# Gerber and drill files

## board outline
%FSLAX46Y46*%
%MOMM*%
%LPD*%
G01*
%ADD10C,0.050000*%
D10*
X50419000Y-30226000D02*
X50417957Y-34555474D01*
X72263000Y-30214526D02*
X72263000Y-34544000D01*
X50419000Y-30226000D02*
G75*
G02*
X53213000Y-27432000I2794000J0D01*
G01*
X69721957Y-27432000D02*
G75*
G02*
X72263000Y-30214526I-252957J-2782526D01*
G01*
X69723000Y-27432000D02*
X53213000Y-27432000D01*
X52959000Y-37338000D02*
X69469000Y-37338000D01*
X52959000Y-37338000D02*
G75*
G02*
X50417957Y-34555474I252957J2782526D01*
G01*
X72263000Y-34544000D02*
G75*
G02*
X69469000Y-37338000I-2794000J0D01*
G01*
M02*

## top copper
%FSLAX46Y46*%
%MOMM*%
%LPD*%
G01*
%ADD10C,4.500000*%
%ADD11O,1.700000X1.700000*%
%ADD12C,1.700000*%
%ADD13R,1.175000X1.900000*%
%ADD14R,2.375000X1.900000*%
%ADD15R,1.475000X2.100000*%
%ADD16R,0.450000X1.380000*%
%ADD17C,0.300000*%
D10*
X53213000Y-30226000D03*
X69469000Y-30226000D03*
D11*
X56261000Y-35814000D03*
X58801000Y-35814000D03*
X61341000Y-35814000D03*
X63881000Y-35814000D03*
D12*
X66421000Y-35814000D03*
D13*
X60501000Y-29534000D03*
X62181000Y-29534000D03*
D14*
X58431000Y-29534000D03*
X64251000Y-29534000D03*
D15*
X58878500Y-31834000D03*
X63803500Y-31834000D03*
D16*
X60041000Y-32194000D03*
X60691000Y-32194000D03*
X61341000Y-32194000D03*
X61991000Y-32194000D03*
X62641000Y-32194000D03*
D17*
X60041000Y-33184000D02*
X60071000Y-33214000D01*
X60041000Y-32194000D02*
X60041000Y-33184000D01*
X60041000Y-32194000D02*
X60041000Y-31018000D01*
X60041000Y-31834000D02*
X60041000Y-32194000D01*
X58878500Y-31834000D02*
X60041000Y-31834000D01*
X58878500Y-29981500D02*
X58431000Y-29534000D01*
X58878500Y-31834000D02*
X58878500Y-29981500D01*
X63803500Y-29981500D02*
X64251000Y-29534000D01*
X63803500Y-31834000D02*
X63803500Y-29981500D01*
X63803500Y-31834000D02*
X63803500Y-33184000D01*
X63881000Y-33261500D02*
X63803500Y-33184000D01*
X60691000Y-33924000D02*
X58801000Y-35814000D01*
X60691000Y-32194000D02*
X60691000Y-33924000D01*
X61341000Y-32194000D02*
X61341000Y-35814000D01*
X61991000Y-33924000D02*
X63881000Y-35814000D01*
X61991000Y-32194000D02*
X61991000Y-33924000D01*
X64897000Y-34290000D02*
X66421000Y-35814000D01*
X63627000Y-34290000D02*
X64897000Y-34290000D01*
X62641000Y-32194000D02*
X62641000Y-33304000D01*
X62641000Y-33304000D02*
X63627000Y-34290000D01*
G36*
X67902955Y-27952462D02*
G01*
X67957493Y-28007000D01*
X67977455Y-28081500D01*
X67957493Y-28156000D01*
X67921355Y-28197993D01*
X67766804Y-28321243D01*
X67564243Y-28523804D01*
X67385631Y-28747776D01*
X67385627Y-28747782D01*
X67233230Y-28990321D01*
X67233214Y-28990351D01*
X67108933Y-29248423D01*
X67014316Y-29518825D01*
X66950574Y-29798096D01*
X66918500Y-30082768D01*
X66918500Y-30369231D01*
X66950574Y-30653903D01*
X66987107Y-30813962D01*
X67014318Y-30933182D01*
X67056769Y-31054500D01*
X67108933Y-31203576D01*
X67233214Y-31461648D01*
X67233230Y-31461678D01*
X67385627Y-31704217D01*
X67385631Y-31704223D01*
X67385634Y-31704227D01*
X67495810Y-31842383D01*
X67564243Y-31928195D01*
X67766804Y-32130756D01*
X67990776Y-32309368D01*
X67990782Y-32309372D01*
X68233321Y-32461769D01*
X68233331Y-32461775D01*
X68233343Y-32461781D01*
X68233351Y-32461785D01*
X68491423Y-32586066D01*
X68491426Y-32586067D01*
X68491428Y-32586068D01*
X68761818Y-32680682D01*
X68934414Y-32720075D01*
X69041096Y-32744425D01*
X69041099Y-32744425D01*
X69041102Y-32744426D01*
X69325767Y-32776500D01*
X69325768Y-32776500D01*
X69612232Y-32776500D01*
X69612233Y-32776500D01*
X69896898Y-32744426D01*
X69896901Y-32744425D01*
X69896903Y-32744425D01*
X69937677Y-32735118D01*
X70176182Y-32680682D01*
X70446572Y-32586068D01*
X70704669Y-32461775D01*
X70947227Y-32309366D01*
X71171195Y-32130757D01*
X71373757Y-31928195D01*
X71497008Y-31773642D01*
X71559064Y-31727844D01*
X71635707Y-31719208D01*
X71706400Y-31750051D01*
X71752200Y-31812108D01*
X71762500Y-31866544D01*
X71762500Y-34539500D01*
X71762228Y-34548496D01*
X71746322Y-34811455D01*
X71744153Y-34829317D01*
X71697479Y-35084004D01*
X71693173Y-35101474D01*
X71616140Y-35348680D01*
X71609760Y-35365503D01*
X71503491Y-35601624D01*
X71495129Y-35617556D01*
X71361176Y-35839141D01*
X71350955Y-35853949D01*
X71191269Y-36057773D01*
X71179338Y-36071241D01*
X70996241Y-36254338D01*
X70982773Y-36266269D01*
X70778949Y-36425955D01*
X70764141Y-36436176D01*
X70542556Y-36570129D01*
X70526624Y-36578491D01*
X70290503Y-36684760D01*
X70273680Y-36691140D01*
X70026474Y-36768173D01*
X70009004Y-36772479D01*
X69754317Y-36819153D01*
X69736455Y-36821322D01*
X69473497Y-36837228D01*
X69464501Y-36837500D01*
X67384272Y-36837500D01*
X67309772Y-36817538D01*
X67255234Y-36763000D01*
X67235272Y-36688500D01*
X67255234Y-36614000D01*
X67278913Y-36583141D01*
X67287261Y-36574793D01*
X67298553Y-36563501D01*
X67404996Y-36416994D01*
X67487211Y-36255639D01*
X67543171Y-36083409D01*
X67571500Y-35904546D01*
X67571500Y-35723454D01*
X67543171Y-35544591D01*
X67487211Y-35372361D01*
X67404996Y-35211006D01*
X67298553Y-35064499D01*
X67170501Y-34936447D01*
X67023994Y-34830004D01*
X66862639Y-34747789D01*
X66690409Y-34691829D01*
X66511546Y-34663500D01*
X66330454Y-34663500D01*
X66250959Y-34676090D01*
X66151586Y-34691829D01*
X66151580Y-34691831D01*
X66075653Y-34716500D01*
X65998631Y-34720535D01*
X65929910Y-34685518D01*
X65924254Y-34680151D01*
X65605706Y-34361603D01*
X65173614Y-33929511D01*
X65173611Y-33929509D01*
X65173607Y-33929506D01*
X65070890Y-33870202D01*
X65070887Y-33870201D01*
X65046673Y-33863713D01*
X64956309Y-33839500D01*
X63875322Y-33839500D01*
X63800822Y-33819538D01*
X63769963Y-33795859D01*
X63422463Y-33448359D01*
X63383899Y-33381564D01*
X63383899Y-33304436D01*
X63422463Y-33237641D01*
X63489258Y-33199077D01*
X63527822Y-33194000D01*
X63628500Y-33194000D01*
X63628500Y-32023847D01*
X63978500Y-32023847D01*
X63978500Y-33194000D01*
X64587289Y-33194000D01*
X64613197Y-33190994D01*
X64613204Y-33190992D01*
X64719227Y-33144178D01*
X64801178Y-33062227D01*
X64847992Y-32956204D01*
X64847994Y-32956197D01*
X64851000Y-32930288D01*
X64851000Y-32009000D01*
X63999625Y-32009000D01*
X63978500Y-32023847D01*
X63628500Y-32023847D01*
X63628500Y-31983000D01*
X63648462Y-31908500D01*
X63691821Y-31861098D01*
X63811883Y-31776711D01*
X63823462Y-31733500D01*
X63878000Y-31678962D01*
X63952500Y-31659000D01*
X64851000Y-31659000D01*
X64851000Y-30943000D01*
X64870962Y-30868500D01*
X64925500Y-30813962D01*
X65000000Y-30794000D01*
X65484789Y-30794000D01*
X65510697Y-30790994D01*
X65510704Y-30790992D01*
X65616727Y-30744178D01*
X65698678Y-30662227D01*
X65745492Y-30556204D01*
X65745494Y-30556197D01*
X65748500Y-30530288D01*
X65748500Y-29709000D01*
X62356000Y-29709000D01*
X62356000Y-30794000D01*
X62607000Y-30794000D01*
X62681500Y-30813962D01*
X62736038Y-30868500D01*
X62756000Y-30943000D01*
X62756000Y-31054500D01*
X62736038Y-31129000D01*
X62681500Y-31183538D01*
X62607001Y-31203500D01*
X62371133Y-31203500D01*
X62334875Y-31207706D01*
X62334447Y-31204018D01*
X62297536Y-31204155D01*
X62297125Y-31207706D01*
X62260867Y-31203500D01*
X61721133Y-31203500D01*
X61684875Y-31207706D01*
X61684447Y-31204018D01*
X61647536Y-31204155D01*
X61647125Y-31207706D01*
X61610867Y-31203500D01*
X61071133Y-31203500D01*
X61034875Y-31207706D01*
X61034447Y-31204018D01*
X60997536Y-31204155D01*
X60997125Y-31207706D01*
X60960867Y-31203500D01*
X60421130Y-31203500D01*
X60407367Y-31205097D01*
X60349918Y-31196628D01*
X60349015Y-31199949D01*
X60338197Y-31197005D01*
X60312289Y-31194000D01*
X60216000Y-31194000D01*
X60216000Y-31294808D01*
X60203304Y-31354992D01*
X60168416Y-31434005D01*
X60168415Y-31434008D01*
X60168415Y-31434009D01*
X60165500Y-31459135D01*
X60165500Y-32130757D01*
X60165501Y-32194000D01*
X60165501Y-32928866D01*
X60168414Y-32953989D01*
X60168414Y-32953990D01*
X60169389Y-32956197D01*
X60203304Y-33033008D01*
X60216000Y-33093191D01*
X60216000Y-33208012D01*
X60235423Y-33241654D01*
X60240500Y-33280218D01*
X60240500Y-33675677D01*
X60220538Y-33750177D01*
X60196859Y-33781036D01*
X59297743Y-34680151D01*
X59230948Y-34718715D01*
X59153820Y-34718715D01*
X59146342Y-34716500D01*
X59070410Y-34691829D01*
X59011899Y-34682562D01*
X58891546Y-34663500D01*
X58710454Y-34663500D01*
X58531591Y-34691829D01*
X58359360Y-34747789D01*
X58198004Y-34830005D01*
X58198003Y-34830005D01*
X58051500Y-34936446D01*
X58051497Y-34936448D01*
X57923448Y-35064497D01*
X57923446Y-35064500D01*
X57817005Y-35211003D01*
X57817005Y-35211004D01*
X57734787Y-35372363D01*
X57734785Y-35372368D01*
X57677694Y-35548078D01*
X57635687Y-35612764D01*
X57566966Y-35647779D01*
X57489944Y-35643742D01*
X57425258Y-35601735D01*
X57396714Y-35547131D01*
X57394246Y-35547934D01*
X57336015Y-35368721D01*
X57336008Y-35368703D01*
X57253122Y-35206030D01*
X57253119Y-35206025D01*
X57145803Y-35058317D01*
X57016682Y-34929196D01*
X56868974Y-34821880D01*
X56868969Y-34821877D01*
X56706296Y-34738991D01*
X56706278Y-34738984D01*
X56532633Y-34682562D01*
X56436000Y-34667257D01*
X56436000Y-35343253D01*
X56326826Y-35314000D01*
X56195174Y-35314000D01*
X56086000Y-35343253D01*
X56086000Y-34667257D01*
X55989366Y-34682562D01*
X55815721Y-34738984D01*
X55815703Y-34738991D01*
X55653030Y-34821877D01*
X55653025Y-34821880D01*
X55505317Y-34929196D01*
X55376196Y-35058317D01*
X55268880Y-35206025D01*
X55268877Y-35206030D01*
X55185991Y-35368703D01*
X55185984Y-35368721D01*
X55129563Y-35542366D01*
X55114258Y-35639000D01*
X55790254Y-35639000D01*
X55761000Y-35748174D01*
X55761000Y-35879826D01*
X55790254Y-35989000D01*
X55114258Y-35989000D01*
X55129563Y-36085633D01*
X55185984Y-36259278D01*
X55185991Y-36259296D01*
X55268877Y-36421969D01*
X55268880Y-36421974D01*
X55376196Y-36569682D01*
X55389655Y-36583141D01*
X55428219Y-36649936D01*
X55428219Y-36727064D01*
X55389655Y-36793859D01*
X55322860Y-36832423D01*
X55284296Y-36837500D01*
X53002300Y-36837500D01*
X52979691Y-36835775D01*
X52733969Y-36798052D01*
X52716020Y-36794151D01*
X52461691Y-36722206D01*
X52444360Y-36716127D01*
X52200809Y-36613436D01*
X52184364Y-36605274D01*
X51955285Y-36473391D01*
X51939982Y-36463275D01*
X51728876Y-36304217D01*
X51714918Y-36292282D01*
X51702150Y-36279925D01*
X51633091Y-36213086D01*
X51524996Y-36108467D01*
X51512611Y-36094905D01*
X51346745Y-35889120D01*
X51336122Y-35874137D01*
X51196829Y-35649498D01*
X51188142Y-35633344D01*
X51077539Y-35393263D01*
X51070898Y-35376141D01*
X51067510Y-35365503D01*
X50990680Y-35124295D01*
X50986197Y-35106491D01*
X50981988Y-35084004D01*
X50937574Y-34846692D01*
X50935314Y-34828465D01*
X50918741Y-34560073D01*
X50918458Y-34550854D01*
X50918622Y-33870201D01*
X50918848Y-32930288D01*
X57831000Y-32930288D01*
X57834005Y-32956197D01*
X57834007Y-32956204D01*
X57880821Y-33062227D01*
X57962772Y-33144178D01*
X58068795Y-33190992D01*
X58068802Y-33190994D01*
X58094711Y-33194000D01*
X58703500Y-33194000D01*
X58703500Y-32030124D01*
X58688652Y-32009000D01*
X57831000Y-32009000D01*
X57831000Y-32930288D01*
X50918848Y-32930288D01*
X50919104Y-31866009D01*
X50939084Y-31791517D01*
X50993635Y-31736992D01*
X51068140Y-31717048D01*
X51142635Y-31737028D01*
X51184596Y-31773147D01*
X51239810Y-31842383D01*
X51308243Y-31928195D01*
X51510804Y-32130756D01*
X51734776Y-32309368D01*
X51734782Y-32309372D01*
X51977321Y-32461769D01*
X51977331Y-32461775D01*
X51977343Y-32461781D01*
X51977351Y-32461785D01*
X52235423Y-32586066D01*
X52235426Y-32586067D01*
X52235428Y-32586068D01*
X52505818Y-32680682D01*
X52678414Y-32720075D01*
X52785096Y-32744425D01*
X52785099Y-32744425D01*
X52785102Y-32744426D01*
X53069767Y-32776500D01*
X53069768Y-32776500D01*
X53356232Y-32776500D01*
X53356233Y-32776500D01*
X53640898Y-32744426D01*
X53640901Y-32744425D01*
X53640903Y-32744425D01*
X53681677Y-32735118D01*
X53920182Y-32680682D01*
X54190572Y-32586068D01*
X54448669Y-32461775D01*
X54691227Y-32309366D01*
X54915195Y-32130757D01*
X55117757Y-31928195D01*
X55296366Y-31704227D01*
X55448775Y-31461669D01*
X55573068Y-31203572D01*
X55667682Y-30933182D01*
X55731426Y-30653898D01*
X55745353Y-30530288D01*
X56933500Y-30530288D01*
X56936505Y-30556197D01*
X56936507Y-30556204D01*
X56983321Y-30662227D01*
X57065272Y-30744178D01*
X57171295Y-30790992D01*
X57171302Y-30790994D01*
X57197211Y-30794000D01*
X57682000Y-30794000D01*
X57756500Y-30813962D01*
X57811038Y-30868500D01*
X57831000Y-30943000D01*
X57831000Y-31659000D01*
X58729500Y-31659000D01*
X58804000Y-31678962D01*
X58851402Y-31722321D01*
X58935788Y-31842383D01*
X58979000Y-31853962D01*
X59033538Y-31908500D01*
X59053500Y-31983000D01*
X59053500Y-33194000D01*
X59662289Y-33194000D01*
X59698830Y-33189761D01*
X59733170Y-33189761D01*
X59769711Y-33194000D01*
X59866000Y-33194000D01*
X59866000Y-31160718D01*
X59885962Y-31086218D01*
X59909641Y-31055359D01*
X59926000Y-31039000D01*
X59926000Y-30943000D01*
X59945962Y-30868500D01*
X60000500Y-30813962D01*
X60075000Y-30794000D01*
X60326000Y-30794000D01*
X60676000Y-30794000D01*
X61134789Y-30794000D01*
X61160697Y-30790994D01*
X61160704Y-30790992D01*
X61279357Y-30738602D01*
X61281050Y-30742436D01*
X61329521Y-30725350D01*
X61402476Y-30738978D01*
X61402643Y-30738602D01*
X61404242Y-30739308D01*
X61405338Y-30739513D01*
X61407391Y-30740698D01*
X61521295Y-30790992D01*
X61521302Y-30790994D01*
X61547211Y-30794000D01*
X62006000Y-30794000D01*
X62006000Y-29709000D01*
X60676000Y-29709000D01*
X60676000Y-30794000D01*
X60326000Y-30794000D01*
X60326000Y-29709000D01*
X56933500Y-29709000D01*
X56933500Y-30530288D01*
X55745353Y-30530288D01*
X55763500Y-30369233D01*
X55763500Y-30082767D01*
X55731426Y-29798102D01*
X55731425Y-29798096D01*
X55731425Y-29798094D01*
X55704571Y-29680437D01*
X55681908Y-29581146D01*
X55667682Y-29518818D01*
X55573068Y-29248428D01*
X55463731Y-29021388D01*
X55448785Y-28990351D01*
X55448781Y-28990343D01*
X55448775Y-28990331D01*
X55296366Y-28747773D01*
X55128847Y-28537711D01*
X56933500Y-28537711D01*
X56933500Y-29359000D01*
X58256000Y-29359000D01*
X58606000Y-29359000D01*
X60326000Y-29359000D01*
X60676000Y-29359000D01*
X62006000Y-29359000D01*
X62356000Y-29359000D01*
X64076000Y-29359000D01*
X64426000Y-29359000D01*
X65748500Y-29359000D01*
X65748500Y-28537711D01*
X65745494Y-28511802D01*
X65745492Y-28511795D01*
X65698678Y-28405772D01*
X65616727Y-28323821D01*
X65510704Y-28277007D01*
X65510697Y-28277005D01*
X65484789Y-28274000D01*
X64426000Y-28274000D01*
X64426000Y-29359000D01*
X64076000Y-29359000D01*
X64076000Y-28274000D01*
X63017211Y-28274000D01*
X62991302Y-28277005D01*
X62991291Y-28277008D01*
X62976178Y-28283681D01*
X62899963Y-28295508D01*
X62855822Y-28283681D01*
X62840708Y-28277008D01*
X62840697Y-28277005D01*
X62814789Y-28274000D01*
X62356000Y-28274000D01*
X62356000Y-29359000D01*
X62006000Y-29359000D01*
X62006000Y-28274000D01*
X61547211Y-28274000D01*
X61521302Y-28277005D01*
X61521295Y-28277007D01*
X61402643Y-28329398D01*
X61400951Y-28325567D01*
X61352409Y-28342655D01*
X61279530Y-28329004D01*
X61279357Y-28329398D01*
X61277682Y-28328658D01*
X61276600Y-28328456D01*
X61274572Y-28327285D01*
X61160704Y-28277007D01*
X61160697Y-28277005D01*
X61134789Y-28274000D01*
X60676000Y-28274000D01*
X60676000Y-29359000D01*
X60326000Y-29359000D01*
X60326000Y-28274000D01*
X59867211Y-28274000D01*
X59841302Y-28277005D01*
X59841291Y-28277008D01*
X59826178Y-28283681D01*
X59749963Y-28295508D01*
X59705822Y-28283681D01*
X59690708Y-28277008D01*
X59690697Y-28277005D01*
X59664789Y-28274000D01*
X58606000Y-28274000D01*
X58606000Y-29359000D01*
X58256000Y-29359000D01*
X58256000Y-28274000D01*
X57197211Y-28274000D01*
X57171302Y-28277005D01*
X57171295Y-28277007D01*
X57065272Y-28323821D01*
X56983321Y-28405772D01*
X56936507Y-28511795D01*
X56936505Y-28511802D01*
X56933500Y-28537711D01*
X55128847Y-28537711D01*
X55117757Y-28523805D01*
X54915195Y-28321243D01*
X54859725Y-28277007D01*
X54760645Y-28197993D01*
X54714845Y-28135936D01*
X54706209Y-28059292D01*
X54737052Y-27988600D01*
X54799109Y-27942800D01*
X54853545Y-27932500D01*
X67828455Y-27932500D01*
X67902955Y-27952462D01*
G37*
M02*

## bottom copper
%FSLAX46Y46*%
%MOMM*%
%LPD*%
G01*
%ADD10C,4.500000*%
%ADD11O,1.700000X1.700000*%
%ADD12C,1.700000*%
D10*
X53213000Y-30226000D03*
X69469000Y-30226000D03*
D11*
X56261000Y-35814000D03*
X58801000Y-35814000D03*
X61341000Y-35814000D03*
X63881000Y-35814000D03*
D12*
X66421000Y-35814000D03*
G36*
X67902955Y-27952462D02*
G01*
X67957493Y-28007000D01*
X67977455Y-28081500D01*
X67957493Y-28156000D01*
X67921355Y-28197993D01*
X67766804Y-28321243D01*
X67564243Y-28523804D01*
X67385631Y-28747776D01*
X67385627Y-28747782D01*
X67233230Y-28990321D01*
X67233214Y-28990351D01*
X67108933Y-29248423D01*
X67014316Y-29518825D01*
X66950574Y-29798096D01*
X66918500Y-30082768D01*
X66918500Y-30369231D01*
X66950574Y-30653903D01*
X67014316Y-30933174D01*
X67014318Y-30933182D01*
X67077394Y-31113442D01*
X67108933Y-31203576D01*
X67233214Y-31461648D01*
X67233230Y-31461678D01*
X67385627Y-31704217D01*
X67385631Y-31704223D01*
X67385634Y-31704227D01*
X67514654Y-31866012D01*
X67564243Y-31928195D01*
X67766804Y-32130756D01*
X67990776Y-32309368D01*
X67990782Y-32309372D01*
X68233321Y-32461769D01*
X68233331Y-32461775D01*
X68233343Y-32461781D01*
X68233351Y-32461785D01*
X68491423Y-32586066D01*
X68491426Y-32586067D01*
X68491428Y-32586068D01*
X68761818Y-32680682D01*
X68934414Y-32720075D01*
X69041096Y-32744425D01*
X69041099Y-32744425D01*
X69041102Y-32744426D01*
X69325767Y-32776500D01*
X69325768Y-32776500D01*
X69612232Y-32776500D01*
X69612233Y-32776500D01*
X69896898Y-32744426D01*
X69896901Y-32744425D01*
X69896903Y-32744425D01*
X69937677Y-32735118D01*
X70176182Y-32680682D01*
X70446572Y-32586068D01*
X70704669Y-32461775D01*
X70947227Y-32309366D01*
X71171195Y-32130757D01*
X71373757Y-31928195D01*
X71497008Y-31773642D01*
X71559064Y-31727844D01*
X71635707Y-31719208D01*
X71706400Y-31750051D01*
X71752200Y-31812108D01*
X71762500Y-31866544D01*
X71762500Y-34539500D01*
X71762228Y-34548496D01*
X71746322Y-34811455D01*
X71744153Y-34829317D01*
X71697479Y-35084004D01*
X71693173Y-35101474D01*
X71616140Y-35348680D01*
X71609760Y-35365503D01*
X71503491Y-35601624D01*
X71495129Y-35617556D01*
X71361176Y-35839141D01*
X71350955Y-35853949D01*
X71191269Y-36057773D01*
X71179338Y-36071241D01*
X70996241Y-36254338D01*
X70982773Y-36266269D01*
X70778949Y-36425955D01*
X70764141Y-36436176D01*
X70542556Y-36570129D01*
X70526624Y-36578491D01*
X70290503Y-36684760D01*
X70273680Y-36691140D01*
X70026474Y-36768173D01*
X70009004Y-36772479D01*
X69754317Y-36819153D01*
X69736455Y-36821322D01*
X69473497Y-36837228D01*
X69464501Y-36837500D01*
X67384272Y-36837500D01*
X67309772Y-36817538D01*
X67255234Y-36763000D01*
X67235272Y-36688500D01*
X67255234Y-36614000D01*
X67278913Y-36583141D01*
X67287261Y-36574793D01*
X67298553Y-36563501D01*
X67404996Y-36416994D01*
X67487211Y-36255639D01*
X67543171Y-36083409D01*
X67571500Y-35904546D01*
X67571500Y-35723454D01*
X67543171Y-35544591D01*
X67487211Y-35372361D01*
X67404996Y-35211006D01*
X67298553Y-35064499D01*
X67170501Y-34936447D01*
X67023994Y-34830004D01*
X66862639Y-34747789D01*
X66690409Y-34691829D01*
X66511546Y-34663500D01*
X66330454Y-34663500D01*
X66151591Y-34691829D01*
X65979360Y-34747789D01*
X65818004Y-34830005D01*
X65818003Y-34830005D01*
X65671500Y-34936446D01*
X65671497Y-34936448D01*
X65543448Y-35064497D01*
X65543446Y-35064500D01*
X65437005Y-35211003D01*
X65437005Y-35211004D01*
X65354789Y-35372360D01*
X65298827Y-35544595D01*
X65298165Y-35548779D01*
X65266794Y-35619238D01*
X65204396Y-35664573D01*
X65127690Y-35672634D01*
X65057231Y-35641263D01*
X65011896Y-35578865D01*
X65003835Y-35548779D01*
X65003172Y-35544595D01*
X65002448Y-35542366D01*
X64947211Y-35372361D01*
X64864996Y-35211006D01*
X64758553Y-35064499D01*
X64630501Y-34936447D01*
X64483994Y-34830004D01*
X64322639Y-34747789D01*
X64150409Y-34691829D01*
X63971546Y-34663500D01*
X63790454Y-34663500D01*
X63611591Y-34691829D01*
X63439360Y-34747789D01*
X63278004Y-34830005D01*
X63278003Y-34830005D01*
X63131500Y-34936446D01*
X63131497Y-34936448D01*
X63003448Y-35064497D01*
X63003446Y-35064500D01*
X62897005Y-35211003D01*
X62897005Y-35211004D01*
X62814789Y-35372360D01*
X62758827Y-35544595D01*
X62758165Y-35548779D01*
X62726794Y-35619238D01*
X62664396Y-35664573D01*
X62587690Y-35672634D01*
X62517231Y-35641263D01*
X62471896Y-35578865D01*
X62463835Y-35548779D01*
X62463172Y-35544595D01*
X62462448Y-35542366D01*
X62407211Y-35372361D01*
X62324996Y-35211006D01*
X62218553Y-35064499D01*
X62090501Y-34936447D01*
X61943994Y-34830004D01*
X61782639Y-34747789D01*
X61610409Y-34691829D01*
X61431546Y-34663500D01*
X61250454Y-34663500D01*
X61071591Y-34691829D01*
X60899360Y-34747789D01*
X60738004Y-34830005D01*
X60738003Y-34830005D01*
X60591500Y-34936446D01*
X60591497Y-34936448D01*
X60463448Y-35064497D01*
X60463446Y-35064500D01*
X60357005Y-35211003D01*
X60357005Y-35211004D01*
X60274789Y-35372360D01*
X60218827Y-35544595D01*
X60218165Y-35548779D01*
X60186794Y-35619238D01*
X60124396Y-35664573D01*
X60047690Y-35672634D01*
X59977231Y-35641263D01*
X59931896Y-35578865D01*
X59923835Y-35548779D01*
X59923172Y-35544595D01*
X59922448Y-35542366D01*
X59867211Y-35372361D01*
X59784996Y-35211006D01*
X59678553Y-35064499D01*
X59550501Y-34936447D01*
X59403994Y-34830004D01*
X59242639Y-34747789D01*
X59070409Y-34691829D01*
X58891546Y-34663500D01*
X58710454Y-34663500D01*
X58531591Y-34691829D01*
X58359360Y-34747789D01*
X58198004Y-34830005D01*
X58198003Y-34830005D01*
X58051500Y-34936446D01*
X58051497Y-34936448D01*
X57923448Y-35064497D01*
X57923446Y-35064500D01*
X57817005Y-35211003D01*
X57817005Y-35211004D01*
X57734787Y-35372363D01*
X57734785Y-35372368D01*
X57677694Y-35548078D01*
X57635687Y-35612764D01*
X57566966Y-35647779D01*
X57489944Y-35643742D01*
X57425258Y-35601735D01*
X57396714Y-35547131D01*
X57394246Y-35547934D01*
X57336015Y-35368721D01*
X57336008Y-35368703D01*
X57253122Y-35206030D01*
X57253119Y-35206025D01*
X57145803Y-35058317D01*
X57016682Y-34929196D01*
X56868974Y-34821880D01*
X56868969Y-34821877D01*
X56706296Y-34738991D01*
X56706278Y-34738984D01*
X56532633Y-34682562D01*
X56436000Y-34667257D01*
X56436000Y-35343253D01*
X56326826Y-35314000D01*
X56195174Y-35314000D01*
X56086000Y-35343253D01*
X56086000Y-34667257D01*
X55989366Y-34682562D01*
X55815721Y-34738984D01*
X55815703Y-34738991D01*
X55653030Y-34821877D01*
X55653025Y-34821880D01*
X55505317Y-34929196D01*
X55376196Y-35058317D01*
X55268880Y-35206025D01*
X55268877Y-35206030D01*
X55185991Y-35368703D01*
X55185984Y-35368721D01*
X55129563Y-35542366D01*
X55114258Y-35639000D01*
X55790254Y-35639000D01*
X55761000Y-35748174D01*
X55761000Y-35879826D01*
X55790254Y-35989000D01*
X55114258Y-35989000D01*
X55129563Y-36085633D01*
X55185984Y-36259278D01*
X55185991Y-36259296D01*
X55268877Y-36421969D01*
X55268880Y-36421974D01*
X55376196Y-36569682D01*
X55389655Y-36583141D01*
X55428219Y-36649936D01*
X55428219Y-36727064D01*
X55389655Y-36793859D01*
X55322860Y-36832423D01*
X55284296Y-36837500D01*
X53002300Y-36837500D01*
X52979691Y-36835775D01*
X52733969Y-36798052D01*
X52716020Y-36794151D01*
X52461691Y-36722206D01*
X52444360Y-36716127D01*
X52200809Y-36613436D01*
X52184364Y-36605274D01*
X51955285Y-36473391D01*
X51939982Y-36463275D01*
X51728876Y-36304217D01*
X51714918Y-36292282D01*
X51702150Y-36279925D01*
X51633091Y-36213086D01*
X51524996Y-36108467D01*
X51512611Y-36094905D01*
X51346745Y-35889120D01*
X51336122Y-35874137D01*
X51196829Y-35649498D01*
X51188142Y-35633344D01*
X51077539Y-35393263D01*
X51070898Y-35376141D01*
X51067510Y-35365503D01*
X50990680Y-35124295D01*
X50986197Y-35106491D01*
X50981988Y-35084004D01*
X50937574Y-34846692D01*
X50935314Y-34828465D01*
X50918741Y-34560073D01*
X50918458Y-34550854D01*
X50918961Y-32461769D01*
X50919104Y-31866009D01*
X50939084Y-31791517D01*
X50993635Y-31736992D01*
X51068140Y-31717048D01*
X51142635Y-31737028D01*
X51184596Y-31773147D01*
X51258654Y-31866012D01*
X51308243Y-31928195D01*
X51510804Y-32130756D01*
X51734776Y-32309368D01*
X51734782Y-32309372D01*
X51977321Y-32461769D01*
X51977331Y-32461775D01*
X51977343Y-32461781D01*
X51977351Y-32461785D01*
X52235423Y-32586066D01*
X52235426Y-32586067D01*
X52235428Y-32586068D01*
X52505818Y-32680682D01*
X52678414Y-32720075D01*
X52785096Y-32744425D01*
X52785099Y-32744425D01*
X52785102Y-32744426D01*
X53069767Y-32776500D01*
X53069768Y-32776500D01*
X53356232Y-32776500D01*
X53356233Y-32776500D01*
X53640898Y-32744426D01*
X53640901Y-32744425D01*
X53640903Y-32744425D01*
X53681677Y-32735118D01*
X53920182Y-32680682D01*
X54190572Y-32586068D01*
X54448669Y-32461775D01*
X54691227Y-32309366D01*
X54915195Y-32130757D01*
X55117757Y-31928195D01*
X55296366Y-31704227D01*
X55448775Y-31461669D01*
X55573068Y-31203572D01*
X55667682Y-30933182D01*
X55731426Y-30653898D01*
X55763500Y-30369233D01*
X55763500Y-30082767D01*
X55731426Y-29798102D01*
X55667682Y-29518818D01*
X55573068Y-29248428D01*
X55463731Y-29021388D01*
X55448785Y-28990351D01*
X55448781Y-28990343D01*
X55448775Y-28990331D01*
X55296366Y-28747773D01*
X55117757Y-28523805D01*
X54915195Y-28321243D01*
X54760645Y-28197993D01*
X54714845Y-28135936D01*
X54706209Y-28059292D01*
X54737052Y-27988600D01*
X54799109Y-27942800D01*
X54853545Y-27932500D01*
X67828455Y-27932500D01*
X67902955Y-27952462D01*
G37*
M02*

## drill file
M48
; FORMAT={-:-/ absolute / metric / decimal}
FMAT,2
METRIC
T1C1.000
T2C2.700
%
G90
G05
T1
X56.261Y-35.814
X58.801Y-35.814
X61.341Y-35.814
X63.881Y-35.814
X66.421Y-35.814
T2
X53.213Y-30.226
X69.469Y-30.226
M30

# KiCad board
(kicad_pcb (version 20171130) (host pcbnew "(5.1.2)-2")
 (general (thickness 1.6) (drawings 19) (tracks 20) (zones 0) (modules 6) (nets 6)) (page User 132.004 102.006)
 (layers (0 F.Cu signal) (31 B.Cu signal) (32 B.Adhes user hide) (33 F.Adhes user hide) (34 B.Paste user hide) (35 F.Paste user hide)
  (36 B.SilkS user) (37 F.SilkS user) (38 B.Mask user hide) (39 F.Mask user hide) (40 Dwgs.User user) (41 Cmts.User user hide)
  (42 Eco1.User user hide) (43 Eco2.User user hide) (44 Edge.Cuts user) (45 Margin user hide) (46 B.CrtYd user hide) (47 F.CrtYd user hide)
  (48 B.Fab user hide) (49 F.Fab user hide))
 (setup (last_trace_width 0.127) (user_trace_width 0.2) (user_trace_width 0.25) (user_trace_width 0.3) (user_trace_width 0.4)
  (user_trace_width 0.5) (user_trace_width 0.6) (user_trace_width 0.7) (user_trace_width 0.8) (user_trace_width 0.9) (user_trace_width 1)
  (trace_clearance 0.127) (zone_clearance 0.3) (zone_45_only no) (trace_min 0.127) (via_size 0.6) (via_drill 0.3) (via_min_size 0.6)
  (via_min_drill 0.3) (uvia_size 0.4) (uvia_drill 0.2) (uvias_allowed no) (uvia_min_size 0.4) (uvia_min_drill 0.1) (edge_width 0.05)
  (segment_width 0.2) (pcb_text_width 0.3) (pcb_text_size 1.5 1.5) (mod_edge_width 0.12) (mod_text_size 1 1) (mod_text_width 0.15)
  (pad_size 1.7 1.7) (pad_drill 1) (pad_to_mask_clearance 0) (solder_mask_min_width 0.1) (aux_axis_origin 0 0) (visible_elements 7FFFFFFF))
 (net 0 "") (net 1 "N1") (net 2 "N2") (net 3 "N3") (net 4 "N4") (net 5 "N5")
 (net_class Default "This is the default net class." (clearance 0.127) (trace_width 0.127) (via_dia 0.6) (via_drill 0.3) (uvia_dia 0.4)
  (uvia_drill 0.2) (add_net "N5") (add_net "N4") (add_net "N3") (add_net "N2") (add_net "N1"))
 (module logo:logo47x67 (layer B.Cu) (at 61.341 30.226 180)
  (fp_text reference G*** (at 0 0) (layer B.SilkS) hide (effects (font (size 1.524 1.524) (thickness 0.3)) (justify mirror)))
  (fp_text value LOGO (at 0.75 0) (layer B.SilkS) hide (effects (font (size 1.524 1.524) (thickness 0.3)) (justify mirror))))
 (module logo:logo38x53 (layer F.Cu) (at 53.213 34.798)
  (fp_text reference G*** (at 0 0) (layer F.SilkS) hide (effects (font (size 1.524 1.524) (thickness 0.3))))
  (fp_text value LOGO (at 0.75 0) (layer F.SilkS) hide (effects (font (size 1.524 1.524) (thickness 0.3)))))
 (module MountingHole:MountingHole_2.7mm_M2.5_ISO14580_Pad (layer F.Cu) (at 53.213 30.226 270)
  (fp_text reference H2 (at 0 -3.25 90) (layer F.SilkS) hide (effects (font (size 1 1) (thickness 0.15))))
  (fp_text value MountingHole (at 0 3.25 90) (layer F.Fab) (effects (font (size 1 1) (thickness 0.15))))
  (pad 1 thru_hole circle (at 0 0 270) (size 4.5 4.5) (drill 2.7) (layers *.Cu *.Mask)))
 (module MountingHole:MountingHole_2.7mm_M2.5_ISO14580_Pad (layer F.Cu) (at 69.469 30.226 270)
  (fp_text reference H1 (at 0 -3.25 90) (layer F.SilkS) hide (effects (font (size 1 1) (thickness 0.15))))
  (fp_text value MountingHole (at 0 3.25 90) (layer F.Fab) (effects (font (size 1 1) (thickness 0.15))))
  (pad 1 thru_hole circle (at 0 0 270) (size 4.5 4.5) (drill 2.7) (layers *.Cu *.Mask)))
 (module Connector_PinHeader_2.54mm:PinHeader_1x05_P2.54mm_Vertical (layer B.Cu) (at 66.421 35.814 90)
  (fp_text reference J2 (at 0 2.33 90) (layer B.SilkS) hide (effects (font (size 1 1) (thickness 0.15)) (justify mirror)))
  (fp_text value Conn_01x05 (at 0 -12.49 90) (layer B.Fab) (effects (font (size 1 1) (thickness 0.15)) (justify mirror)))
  (pad 5 thru_hole oval (at 0 -10.16 90) (size 1.7 1.7) (drill 1) (layers *.Cu *.Mask) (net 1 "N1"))
  (pad 4 thru_hole oval (at 0 -7.62 90) (size 1.7 1.7) (drill 1) (layers *.Cu *.Mask) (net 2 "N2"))
  (pad 3 thru_hole oval (at 0 -5.08 90) (size 1.7 1.7) (drill 1) (layers *.Cu *.Mask) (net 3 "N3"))
  (pad 2 thru_hole oval (at 0 -2.54 90) (size 1.7 1.7) (drill 1) (layers *.Cu *.Mask) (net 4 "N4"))
  (pad 1 thru_hole circle (at 0 0 90) (size 1.7 1.7) (drill 1) (layers *.Cu *.Mask) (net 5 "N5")))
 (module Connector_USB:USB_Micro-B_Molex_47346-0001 (layer F.Cu) (at 61.341 30.734 180)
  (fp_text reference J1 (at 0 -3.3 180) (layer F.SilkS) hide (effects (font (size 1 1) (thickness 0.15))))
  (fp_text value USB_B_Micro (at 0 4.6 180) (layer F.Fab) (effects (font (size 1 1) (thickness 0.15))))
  (pad 6 smd rect (at 0.84 1.2 180) (size 1.175 1.9) (layers F.Cu F.Paste F.Mask) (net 1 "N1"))
  (pad 6 smd rect (at -0.84 1.2 180) (size 1.175 1.9) (layers F.Cu F.Paste F.Mask) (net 1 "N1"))
  (pad 6 smd rect (at 2.91 1.2 180) (size 2.375 1.9) (layers F.Cu F.Paste F.Mask) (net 1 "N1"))
  (pad 6 smd rect (at -2.91 1.2 180) (size 2.375 1.9) (layers F.Cu F.Paste F.Mask) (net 1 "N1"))
  (pad 6 smd rect (at 2.4625 -1.1 180) (size 1.475 2.1) (layers F.Cu F.Paste F.Mask) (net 1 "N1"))
  (pad 6 smd rect (at -2.4625 -1.1 180) (size 1.475 2.1) (layers F.Cu F.Paste F.Mask) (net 1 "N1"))
  (pad 5 smd rect (at 1.3 -1.46 180) (size 0.45 1.38) (layers F.Cu F.Paste F.Mask) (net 1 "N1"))
  (pad 4 smd rect (at 0.65 -1.46 180) (size 0.45 1.38) (layers F.Cu F.Paste F.Mask) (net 2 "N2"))
  (pad 3 smd rect (at 0 -1.46 180) (size 0.45 1.38) (layers F.Cu F.Paste F.Mask) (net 3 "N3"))
  (pad 2 smd rect (at -0.65 -1.46 180) (size 0.45 1.38) (layers F.Cu F.Paste F.Mask) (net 4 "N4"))
  (pad 1 smd rect (at -1.3 -1.46 180) (size 0.45 1.38) (layers F.Cu F.Paste F.Mask) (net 5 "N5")))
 (gr_line (start 50.419 30.226) (end 50.417957 34.555474) (layer Edge.Cuts) (width 0.05))
 (gr_line (start 72.263 30.214526) (end 72.263 34.544) (layer Edge.Cuts) (width 0.05))
 (gr_arc (start 53.213 30.226) (end 53.213 27.432) (angle -90) (layer Edge.Cuts) (width 0.05))
 (gr_arc (start 69.469 30.214526) (end 72.263 30.214526) (angle -84.80557109) (layer Edge.Cuts) (width 0.05))
 (gr_line (start 69.723 27.432) (end 53.213 27.432) (layer Edge.Cuts) (width 0.05))
 (gr_line (start 52.959 37.338) (end 69.469 37.338) (layer Edge.Cuts) (width 0.05))
 (gr_arc (start 53.211957 34.555474) (end 50.417957 34.555474) (angle -84.80557109) (layer Edge.Cuts) (width 0.05))
 (gr_arc (start 69.469 34.544) (end 69.469 37.338) (angle -90) (layer Edge.Cuts) (width 0.05))
 (segment (start 60.041 33.184) (end 60.071 33.214) (width 0.3) (layer F.Cu) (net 1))
 (segment (start 60.041 32.194) (end 60.041 33.184) (width 0.3) (layer F.Cu) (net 1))
 (segment (start 60.041 32.194) (end 60.041 31.018) (width 0.3) (layer F.Cu) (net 1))
 (segment (start 60.041 31.834) (end 60.041 32.194) (width 0.3) (layer F.Cu) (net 1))
 (segment (start 58.8785 31.834) (end 60.041 31.834) (width 0.3) (layer F.Cu) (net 1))
 (segment (start 58.8785 29.9815) (end 58.431 29.534) (width 0.3) (layer F.Cu) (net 1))
 (segment (start 58.8785 31.834) (end 58.8785 29.9815) (width 0.3) (layer F.Cu) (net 1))
 (segment (start 63.8035 29.9815) (end 64.251 29.534) (width 0.3) (layer F.Cu) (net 1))
 (segment (start 63.8035 31.834) (end 63.8035 29.9815) (width 0.3) (layer F.Cu) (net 1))
 (segment (start 63.8035 31.834) (end 63.8035 33.184) (width 0.3) (layer F.Cu) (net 1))
 (segment (start 63.881 33.2615) (end 63.8035 33.184) (width 0.3) (layer F.Cu) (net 1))
 (segment (start 60.691 33.924) (end 58.801 35.814) (width 0.3) (layer F.Cu) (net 2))
 (segment (start 60.691 32.194) (end 60.691 33.924) (width 0.3) (layer F.Cu) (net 2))
 (segment (start 61.341 32.194) (end 61.341 35.814) (width 0.3) (layer F.Cu) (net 3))
 (segment (start 61.991 33.924) (end 63.881 35.814) (width 0.3) (layer F.Cu) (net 4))
 (segment (start 61.991 32.194) (end 61.991 33.924) (width 0.3) (layer F.Cu) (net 4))
 (segment (start 64.897 34.29) (end 66.421 35.814) (width 0.3) (layer F.Cu) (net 5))
 (segment (start 63.627 34.29) (end 64.897 34.29) (width 0.3) (layer F.Cu) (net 5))
 (segment (start 62.641 32.194) (end 62.641 33.304) (width 0.3) (layer F.Cu) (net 5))
 (segment (start 62.641 33.304) (end 63.627 34.29) (width 0.3) (layer F.Cu) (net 5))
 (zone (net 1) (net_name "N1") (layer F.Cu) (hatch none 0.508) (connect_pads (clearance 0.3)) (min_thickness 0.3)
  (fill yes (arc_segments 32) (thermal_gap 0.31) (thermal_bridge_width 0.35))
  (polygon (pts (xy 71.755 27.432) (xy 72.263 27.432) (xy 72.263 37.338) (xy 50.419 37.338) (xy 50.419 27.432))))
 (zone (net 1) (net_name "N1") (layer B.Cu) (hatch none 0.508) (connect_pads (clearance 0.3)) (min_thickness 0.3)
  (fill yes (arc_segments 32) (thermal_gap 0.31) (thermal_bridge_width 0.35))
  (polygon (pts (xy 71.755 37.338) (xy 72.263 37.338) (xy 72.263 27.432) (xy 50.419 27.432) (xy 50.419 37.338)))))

